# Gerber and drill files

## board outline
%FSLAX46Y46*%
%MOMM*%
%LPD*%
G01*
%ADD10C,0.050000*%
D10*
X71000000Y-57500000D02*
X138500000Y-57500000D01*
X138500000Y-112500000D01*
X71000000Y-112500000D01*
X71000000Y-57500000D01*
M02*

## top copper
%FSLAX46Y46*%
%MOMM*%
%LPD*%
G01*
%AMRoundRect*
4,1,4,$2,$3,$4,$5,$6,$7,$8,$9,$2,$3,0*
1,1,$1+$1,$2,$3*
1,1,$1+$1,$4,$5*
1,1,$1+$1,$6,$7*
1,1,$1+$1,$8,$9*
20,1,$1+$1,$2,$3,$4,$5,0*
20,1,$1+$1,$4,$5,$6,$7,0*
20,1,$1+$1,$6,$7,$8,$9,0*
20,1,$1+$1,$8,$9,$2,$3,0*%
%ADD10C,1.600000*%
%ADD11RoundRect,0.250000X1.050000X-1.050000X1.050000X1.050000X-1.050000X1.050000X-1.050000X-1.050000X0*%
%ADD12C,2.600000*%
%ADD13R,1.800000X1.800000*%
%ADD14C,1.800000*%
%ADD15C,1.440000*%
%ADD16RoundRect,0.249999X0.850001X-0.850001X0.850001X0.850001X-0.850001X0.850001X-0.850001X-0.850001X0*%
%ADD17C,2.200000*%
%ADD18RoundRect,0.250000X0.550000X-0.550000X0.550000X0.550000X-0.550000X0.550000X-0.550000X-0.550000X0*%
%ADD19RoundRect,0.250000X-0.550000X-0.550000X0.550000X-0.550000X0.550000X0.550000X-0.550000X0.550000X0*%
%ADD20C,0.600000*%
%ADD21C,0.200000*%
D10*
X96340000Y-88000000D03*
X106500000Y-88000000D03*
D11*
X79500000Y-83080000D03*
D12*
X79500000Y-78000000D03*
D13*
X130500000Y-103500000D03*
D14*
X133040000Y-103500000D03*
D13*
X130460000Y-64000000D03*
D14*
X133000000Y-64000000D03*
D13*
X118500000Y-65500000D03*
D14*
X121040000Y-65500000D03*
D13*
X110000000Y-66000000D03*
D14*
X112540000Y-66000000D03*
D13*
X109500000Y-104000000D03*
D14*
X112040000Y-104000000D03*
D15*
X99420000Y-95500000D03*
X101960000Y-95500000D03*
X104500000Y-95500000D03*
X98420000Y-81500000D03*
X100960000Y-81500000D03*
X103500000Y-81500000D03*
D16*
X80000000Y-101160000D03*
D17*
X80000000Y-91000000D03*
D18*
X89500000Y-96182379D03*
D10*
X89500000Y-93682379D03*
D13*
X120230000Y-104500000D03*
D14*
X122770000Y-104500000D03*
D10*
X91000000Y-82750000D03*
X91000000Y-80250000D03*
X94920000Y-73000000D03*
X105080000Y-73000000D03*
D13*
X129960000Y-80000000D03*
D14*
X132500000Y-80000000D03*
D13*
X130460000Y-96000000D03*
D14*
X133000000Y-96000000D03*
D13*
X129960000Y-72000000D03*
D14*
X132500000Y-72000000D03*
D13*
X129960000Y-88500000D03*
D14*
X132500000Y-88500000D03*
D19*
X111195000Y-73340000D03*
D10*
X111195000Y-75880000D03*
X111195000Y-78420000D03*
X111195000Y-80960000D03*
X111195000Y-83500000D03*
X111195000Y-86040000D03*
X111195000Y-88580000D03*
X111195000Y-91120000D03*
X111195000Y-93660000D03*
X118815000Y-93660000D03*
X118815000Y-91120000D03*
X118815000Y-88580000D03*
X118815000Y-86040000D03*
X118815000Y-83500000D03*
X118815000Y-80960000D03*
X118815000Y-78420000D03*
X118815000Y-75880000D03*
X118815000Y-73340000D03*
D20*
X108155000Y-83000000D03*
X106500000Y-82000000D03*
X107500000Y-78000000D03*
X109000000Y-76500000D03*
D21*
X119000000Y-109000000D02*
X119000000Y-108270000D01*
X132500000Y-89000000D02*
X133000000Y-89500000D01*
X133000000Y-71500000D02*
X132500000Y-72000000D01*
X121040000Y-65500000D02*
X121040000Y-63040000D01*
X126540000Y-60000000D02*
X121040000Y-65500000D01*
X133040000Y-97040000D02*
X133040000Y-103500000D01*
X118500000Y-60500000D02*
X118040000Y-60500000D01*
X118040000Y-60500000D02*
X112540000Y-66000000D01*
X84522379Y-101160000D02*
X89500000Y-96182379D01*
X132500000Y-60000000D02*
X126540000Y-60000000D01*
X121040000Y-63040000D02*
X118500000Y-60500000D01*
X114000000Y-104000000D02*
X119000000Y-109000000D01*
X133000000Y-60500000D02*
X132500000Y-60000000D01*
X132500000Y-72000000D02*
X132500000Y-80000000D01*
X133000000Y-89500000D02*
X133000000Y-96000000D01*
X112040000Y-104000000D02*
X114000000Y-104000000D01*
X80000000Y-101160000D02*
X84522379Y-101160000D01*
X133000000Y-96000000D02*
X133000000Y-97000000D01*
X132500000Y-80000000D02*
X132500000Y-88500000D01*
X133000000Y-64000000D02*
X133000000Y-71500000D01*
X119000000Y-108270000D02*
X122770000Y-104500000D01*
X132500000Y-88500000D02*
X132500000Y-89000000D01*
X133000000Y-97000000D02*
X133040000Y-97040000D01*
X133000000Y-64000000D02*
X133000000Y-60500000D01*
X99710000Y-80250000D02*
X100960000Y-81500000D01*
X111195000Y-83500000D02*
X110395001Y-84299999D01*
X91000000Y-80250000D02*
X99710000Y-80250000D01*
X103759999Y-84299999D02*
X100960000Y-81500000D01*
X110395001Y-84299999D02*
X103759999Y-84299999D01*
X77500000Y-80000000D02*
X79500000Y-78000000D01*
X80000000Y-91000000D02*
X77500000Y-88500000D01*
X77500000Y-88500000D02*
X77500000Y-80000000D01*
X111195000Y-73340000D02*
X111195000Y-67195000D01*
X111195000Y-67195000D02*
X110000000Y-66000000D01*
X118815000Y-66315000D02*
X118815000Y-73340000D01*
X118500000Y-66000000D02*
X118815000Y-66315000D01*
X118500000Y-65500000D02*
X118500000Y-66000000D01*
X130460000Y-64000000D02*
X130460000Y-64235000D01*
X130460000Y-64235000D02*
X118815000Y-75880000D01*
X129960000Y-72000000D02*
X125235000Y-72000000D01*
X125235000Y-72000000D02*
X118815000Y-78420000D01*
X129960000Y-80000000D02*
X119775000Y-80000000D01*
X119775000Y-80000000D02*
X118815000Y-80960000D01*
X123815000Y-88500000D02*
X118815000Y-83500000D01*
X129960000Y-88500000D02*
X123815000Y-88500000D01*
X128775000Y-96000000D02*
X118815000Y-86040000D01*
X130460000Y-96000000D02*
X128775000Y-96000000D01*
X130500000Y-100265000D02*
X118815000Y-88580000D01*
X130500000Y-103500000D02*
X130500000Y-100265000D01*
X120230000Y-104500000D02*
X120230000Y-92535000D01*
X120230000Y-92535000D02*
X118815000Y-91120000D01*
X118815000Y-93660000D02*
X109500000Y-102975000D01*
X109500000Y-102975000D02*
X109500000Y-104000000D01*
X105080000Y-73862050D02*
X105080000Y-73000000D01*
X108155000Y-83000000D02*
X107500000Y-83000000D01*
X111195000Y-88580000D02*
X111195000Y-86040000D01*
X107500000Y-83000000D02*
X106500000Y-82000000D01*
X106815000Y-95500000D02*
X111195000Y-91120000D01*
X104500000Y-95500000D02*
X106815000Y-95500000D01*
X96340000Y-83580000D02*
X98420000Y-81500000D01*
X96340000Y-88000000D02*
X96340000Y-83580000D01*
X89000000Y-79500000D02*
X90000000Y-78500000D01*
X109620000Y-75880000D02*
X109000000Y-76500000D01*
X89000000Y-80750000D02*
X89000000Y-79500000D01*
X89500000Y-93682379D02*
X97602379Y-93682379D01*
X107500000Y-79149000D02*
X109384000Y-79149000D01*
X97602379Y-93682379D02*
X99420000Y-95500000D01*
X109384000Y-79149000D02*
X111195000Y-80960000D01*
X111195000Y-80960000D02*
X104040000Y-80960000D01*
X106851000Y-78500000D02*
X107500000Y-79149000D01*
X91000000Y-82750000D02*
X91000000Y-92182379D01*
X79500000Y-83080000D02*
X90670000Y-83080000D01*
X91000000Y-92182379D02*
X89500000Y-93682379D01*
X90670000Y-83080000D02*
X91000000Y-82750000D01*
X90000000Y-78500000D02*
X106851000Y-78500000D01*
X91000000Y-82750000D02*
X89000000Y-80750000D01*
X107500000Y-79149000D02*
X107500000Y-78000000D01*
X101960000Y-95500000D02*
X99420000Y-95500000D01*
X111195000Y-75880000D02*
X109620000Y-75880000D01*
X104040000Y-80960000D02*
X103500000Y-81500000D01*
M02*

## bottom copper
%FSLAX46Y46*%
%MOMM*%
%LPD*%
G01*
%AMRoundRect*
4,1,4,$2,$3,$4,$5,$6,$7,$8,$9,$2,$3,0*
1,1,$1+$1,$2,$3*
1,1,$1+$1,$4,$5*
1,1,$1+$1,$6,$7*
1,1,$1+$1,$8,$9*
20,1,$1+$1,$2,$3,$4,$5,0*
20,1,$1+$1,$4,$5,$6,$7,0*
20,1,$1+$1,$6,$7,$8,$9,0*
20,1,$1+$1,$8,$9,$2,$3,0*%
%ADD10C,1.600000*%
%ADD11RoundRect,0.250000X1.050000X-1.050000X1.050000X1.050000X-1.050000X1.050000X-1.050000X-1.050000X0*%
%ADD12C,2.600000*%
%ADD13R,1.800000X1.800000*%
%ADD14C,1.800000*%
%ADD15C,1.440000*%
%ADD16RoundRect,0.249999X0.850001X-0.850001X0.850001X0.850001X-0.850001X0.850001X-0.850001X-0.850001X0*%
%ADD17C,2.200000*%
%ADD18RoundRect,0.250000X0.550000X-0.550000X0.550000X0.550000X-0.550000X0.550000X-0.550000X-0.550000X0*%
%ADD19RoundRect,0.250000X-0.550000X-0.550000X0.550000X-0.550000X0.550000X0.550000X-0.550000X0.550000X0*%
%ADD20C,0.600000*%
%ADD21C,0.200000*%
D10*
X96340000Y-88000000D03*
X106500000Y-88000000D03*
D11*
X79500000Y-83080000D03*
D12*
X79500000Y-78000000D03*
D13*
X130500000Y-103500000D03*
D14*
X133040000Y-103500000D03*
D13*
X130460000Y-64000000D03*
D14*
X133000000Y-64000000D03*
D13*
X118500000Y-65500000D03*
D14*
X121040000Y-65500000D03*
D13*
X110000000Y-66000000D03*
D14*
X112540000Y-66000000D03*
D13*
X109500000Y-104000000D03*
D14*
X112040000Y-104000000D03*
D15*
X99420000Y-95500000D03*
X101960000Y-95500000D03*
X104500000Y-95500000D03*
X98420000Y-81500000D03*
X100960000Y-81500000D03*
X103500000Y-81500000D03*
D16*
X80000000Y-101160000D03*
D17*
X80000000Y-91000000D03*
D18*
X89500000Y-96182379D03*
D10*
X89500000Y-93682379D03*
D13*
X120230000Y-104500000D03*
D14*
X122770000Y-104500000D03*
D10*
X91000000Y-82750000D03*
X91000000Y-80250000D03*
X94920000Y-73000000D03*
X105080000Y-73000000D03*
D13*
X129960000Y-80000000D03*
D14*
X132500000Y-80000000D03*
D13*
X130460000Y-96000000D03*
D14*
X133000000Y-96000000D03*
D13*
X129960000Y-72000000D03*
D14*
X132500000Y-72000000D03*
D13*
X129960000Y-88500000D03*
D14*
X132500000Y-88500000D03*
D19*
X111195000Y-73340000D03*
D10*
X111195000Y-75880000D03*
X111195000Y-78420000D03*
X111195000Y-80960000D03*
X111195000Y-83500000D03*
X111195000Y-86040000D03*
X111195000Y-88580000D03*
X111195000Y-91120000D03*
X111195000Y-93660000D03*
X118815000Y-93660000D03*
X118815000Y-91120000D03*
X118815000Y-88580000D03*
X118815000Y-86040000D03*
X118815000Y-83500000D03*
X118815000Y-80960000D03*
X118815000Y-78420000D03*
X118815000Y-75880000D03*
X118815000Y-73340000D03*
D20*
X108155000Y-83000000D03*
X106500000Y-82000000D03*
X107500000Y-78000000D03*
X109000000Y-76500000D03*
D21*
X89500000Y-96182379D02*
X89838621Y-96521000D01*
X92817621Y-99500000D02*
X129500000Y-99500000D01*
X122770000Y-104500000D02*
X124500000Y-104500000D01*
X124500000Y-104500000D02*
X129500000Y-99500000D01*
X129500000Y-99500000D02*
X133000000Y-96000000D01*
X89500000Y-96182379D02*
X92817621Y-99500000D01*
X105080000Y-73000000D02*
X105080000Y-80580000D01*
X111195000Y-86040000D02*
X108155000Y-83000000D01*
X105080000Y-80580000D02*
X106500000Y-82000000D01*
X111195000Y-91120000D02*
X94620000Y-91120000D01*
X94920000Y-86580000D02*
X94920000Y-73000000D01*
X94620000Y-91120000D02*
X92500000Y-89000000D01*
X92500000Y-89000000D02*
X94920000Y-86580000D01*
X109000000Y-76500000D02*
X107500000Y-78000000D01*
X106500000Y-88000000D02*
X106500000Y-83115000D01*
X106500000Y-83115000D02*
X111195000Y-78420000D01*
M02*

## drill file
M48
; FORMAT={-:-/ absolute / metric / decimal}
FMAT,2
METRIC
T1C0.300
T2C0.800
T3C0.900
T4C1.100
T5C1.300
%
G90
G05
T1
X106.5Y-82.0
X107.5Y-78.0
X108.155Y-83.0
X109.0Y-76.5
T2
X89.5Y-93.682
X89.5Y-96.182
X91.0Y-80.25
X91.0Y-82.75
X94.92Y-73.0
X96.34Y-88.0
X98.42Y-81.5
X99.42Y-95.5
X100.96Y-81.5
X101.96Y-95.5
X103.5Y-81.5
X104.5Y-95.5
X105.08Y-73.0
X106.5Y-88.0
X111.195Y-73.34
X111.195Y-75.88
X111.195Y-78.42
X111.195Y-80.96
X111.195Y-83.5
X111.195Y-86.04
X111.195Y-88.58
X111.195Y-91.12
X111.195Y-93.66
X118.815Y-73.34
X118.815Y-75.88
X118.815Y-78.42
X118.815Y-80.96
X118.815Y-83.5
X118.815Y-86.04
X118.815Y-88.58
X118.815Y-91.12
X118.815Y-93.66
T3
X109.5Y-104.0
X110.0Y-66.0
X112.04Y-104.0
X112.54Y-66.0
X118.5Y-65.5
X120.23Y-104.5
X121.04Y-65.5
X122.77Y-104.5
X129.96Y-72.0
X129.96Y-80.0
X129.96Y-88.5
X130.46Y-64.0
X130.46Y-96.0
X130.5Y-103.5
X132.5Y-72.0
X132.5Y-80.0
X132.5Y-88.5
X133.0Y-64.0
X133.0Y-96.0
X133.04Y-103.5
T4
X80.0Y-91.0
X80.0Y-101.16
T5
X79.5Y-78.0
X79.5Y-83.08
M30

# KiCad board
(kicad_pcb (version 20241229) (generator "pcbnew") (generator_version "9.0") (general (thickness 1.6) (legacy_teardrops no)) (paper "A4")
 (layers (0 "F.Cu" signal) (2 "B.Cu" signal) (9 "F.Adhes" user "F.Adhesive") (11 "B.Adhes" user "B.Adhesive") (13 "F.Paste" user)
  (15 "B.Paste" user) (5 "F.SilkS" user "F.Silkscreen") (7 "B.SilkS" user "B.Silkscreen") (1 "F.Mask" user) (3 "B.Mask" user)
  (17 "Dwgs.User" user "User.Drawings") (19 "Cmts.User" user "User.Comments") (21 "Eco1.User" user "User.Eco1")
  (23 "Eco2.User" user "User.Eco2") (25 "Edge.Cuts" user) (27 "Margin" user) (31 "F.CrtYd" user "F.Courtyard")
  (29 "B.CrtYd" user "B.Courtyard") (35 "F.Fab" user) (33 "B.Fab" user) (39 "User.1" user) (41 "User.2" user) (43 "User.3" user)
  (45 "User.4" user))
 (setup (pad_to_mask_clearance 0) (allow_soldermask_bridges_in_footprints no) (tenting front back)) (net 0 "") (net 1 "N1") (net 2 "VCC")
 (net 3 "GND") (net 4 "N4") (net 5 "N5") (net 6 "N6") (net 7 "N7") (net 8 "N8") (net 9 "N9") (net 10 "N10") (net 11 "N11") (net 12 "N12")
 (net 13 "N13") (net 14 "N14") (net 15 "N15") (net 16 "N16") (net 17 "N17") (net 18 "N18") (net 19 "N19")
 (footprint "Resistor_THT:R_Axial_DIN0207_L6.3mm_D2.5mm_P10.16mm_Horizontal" (layer "F.Cu") (at 96.34 88)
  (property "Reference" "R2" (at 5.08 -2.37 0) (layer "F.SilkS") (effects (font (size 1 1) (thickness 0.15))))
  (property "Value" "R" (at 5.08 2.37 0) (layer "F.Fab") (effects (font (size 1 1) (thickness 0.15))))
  (pad "1" thru_hole circle (at 0 0) (size 1.6 1.6) (drill 0.8) (layers "*.Cu" "*.Mask") (remove_unused_layers no) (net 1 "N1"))
  (pad "2" thru_hole circle (at 10.16 0) (size 1.6 1.6) (drill 0.8) (layers "*.Cu" "*.Mask") (remove_unused_layers no) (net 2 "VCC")))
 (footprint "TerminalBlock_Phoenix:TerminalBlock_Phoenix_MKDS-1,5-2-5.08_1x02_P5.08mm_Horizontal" (layer "F.Cu") (at 79.5 83.08 90)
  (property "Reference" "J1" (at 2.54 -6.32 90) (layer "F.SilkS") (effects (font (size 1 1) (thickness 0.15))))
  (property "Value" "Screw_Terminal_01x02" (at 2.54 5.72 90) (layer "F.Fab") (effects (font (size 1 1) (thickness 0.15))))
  (pad "1" thru_hole roundrect (at 0 0 90) (size 2.6 2.6) (drill 1.3) (layers "*.Cu" "*.Mask") (remove_unused_layers no)
   (roundrect_rratio 0.096154) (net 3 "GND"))
  (pad "2" thru_hole circle (at 5.08 0 90) (size 2.6 2.6) (drill 1.3) (layers "*.Cu" "*.Mask") (remove_unused_layers no) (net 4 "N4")))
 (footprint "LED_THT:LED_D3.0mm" (layer "F.Cu") (at 130.5 103.5)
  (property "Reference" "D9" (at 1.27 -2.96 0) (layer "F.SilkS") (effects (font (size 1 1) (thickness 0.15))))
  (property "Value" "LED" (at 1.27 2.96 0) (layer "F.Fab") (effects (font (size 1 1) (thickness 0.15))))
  (pad "1" thru_hole rect (at 0 0) (size 1.8 1.8) (drill 0.9) (layers "*.Cu" "*.Mask") (remove_unused_layers no) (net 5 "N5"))
  (pad "2" thru_hole circle (at 2.54 0) (size 1.8 1.8) (drill 0.9) (layers "*.Cu" "*.Mask") (remove_unused_layers no) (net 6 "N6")))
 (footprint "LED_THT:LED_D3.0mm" (layer "F.Cu") (at 130.46 64)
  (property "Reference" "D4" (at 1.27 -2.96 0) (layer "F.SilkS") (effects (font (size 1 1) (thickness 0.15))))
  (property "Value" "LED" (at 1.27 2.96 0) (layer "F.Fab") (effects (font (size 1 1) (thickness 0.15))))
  (pad "1" thru_hole rect (at 0 0) (size 1.8 1.8) (drill 0.9) (layers "*.Cu" "*.Mask") (remove_unused_layers no) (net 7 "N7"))
  (pad "2" thru_hole circle (at 2.54 0) (size 1.8 1.8) (drill 0.9) (layers "*.Cu" "*.Mask") (remove_unused_layers no) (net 6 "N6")))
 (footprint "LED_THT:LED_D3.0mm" (layer "F.Cu") (at 118.5 65.5)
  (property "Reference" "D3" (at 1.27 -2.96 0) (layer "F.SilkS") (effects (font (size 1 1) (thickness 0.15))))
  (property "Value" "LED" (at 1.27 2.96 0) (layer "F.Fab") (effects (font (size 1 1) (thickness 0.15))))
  (pad "1" thru_hole rect (at 0 0) (size 1.8 1.8) (drill 0.9) (layers "*.Cu" "*.Mask") (remove_unused_layers no) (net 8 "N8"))
  (pad "2" thru_hole circle (at 2.54 0) (size 1.8 1.8) (drill 0.9) (layers "*.Cu" "*.Mask") (remove_unused_layers no) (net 6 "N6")))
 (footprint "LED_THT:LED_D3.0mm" (layer "F.Cu") (at 110 66)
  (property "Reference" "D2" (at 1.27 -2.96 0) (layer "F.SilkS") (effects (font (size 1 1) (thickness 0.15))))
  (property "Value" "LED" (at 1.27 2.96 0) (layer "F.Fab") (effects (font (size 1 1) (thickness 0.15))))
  (pad "1" thru_hole rect (at 0 0) (size 1.8 1.8) (drill 0.9) (layers "*.Cu" "*.Mask") (remove_unused_layers no) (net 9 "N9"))
  (pad "2" thru_hole circle (at 2.54 0) (size 1.8 1.8) (drill 0.9) (layers "*.Cu" "*.Mask") (remove_unused_layers no) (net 6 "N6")))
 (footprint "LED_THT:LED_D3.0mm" (layer "F.Cu") (at 109.5 104)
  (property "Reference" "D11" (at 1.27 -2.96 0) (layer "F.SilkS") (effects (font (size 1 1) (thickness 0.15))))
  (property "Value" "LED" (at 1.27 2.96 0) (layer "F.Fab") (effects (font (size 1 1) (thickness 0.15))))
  (pad "1" thru_hole rect (at 0 0) (size 1.8 1.8) (drill 0.9) (layers "*.Cu" "*.Mask") (remove_unused_layers no) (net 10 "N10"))
  (pad "2" thru_hole circle (at 2.54 0) (size 1.8 1.8) (drill 0.9) (layers "*.Cu" "*.Mask") (remove_unused_layers no) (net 6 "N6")))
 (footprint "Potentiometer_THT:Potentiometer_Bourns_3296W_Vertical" (layer "F.Cu") (at 99.42 95.5 180)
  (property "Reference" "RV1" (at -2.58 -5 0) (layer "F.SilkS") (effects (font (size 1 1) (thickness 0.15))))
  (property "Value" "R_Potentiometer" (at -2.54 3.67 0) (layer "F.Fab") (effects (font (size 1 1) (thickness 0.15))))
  (pad "1" thru_hole circle (at 0 0 180) (size 1.44 1.44) (drill 0.8) (layers "*.Cu" "*.Mask") (remove_unused_layers no) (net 3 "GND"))
  (pad "2" thru_hole circle (at -2.54 0 180) (size 1.44 1.44) (drill 0.8) (layers "*.Cu" "*.Mask") (remove_unused_layers no) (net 3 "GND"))
  (pad "3" thru_hole circle (at -5.08 0 180) (size 1.44 1.44) (drill 0.8) (layers "*.Cu" "*.Mask") (remove_unused_layers no) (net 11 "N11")))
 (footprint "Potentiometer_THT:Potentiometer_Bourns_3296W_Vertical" (layer "F.Cu") (at 98.42 81.5 180)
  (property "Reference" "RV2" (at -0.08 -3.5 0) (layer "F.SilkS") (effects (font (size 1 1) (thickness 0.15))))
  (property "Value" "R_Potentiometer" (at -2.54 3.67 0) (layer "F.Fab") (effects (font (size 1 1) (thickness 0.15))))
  (pad "1" thru_hole circle (at 0 0 180) (size 1.44 1.44) (drill 0.8) (layers "*.Cu" "*.Mask") (remove_unused_layers no) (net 1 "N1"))
  (pad "2" thru_hole circle (at -2.54 0 180) (size 1.44 1.44) (drill 0.8) (layers "*.Cu" "*.Mask") (remove_unused_layers no) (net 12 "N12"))
  (pad "3" thru_hole circle (at -5.08 0 180) (size 1.44 1.44) (drill 0.8) (layers "*.Cu" "*.Mask") (remove_unused_layers no) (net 3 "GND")))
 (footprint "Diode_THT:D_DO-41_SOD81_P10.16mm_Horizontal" (layer "F.Cu") (at 80 101.16 90)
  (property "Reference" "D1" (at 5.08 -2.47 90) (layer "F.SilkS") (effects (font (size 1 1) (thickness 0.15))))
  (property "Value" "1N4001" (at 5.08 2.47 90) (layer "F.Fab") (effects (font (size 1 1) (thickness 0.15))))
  (pad "1" thru_hole roundrect (at 0 0 90) (size 2.2 2.2) (drill 1.1) (layers "*.Cu" "*.Mask") (remove_unused_layers no)
   (roundrect_rratio 0.113636) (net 6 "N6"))
  (pad "2" thru_hole circle (at 10.16 0 90) (size 2.2 2.2) (drill 1.1) (layers "*.Cu" "*.Mask") (remove_unused_layers no) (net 4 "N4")))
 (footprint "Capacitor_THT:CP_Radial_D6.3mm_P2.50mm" (layer "F.Cu") (at 89.5 96.182379 90)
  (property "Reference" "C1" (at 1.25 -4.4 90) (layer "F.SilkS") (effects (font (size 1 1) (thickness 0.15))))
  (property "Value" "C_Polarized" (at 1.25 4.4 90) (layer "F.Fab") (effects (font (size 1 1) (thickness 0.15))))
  (pad "1" thru_hole roundrect (at 0 0 90) (size 1.6 1.6) (drill 0.8) (layers "*.Cu" "*.Mask") (remove_unused_layers no)
   (roundrect_rratio 0.15625) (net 6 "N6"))
  (pad "2" thru_hole circle (at 2.5 0 90) (size 1.6 1.6) (drill 0.8) (layers "*.Cu" "*.Mask") (remove_unused_layers no) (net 3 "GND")))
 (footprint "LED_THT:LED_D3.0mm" (layer "F.Cu") (at 120.23 104.5)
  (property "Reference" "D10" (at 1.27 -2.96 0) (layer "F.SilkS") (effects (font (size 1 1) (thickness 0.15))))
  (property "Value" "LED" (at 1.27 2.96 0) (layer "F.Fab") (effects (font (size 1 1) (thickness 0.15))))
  (pad "1" thru_hole rect (at 0 0) (size 1.8 1.8) (drill 0.9) (layers "*.Cu" "*.Mask") (remove_unused_layers no) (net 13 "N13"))
  (pad "2" thru_hole circle (at 2.54 0) (size 1.8 1.8) (drill 0.9) (layers "*.Cu" "*.Mask") (remove_unused_layers no) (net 6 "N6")))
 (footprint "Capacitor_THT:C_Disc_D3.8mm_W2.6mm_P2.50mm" (layer "F.Cu") (at 91 82.75 90)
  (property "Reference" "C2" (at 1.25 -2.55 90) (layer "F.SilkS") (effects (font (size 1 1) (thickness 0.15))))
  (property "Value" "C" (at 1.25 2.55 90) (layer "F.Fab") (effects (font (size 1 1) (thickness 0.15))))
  (pad "1" thru_hole circle (at 0 0 90) (size 1.6 1.6) (drill 0.8) (layers "*.Cu" "*.Mask") (remove_unused_layers no) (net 3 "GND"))
  (pad "2" thru_hole circle (at 2.5 0 90) (size 1.6 1.6) (drill 0.8) (layers "*.Cu" "*.Mask") (remove_unused_layers no) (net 12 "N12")))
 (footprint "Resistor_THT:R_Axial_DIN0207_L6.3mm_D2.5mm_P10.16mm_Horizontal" (layer "F.Cu") (at 94.92 73)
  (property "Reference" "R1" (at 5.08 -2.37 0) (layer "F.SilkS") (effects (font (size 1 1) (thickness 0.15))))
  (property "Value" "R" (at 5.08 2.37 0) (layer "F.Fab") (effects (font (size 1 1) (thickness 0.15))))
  (pad "1" thru_hole circle (at 0 0) (size 1.6 1.6) (drill 0.8) (layers "*.Cu" "*.Mask") (remove_unused_layers no) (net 11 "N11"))
  (pad "2" thru_hole circle (at 10.16 0) (size 1.6 1.6) (drill 0.8) (layers "*.Cu" "*.Mask") (remove_unused_layers no) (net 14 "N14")))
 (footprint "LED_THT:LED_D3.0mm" (layer "F.Cu") (at 129.96 80)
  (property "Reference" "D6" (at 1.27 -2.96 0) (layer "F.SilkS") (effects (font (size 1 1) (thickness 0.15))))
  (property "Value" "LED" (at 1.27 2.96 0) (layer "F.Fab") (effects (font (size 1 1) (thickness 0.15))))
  (pad "1" thru_hole rect (at 0 0) (size 1.8 1.8) (drill 0.9) (layers "*.Cu" "*.Mask") (remove_unused_layers no) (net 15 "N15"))
  (pad "2" thru_hole circle (at 2.54 0) (size 1.8 1.8) (drill 0.9) (layers "*.Cu" "*.Mask") (remove_unused_layers no) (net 6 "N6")))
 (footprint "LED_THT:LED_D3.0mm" (layer "F.Cu") (at 130.46 96)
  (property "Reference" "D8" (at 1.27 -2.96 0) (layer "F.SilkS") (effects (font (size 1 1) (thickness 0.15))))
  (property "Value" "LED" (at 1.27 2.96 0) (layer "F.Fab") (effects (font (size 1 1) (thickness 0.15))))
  (pad "1" thru_hole rect (at 0 0) (size 1.8 1.8) (drill 0.9) (layers "*.Cu" "*.Mask") (remove_unused_layers no) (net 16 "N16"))
  (pad "2" thru_hole circle (at 2.54 0) (size 1.8 1.8) (drill 0.9) (layers "*.Cu" "*.Mask") (remove_unused_layers no) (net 6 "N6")))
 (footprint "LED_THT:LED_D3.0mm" (layer "F.Cu") (at 129.96 72)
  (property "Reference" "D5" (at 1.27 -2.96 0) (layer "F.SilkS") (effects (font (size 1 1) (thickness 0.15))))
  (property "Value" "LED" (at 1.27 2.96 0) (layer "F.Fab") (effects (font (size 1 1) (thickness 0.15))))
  (pad "1" thru_hole rect (at 0 0) (size 1.8 1.8) (drill 0.9) (layers "*.Cu" "*.Mask") (remove_unused_layers no) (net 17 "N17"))
  (pad "2" thru_hole circle (at 2.54 0) (size 1.8 1.8) (drill 0.9) (layers "*.Cu" "*.Mask") (remove_unused_layers no) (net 6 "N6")))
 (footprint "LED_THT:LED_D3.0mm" (layer "F.Cu") (at 129.96 88.5)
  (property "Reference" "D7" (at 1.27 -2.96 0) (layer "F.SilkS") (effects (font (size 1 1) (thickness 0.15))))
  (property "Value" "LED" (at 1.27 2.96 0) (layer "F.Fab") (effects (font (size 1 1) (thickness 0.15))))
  (pad "1" thru_hole rect (at 0 0) (size 1.8 1.8) (drill 0.9) (layers "*.Cu" "*.Mask") (remove_unused_layers no) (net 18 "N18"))
  (pad "2" thru_hole circle (at 2.54 0) (size 1.8 1.8) (drill 0.9) (layers "*.Cu" "*.Mask") (remove_unused_layers no) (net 6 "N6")))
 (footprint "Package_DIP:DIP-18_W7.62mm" (layer "F.Cu") (at 111.195 73.34)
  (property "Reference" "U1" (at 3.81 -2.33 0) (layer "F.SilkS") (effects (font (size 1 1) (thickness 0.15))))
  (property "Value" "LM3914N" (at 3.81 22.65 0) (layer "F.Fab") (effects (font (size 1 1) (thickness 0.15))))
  (pad "1" thru_hole roundrect (at 0 0) (size 1.6 1.6) (drill 0.8) (layers "*.Cu" "*.Mask") (remove_unused_layers no)
   (roundrect_rratio 0.15625) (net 9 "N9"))
  (pad "2" thru_hole circle (at 0 2.54) (size 1.6 1.6) (drill 0.8) (layers "*.Cu" "*.Mask") (remove_unused_layers no) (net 3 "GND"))
  (pad "3" thru_hole circle (at 0 5.08) (size 1.6 1.6) (drill 0.8) (layers "*.Cu" "*.Mask") (remove_unused_layers no) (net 2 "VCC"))
  (pad "4" thru_hole circle (at 0 7.62) (size 1.6 1.6) (drill 0.8) (layers "*.Cu" "*.Mask") (remove_unused_layers no) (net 3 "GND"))
  (pad "5" thru_hole circle (at 0 10.16) (size 1.6 1.6) (drill 0.8) (layers "*.Cu" "*.Mask") (remove_unused_layers no) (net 12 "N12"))
  (pad "6" thru_hole circle (at 0 12.7) (size 1.6 1.6) (drill 0.8) (layers "*.Cu" "*.Mask") (remove_unused_layers no) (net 14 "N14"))
  (pad "7" thru_hole circle (at 0 15.24) (size 1.6 1.6) (drill 0.8) (layers "*.Cu" "*.Mask") (remove_unused_layers no) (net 14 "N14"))
  (pad "8" thru_hole circle (at 0 17.78) (size 1.6 1.6) (drill 0.8) (layers "*.Cu" "*.Mask") (remove_unused_layers no) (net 11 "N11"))
  (pad "9" thru_hole circle (at 0 20.32) (size 1.6 1.6) (drill 0.8) (layers "*.Cu" "*.Mask") (remove_unused_layers no) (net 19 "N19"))
  (pad "10" thru_hole circle (at 7.62 20.32) (size 1.6 1.6) (drill 0.8) (layers "*.Cu" "*.Mask") (remove_unused_layers no) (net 10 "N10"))
  (pad "11" thru_hole circle (at 7.62 17.78) (size 1.6 1.6) (drill 0.8) (layers "*.Cu" "*.Mask") (remove_unused_layers no) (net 13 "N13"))
  (pad "12" thru_hole circle (at 7.62 15.24) (size 1.6 1.6) (drill 0.8) (layers "*.Cu" "*.Mask") (remove_unused_layers no) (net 5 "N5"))
  (pad "13" thru_hole circle (at 7.62 12.7) (size 1.6 1.6) (drill 0.8) (layers "*.Cu" "*.Mask") (remove_unused_layers no) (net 16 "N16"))
  (pad "14" thru_hole circle (at 7.62 10.16) (size 1.6 1.6) (drill 0.8) (layers "*.Cu" "*.Mask") (remove_unused_layers no) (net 18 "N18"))
  (pad "15" thru_hole circle (at 7.62 7.62) (size 1.6 1.6) (drill 0.8) (layers "*.Cu" "*.Mask") (remove_unused_layers no) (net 15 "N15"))
  (pad "16" thru_hole circle (at 7.62 5.08) (size 1.6 1.6) (drill 0.8) (layers "*.Cu" "*.Mask") (remove_unused_layers no) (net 17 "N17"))
  (pad "17" thru_hole circle (at 7.62 2.54) (size 1.6 1.6) (drill 0.8) (layers "*.Cu" "*.Mask") (remove_unused_layers no) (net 7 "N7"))
  (pad "18" thru_hole circle (at 7.62 0) (size 1.6 1.6) (drill 0.8) (layers "*.Cu" "*.Mask") (remove_unused_layers no) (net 8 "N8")))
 (gr_rect (start 71 57.5) (end 138.5 112.5) (stroke (width 0.05) (type default)) (fill no) (layer "Edge.Cuts"))
 (segment (start 119 109) (end 119 108.27) (width 0.2) (layer "F.Cu") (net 6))
 (segment (start 132.5 89) (end 133 89.5) (width 0.2) (layer "F.Cu") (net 6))
 (segment (start 133 71.5) (end 132.5 72) (width 0.2) (layer "F.Cu") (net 6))
 (segment (start 121.04 65.5) (end 121.04 63.04) (width 0.2) (layer "F.Cu") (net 6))
 (segment (start 126.54 60) (end 121.04 65.5) (width 0.2) (layer "F.Cu") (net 6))
 (segment (start 133.04 97.04) (end 133.04 103.5) (width 0.2) (layer "F.Cu") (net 6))
 (segment (start 118.5 60.5) (end 118.04 60.5) (width 0.2) (layer "F.Cu") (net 6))
 (segment (start 118.04 60.5) (end 112.54 66) (width 0.2) (layer "F.Cu") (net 6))
 (segment (start 84.522379 101.16) (end 89.5 96.182379) (width 0.2) (layer "F.Cu") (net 6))
 (segment (start 132.5 60) (end 126.54 60) (width 0.2) (layer "F.Cu") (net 6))
 (segment (start 121.04 63.04) (end 118.5 60.5) (width 0.2) (layer "F.Cu") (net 6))
 (segment (start 114 104) (end 119 109) (width 0.2) (layer "F.Cu") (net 6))
 (segment (start 133 60.5) (end 132.5 60) (width 0.2) (layer "F.Cu") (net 6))
 (segment (start 132.5 72) (end 132.5 80) (width 0.2) (layer "F.Cu") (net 6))
 (segment (start 133 89.5) (end 133 96) (width 0.2) (layer "F.Cu") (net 6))
 (segment (start 112.04 104) (end 114 104) (width 0.2) (layer "F.Cu") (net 6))
 (segment (start 80 101.16) (end 84.522379 101.16) (width 0.2) (layer "F.Cu") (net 6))
 (segment (start 133 96) (end 133 97) (width 0.2) (layer "F.Cu") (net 6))
 (segment (start 132.5 80) (end 132.5 88.5) (width 0.2) (layer "F.Cu") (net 6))
 (segment (start 133 64) (end 133 71.5) (width 0.2) (layer "F.Cu") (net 6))
 (segment (start 119 108.27) (end 122.77 104.5) (width 0.2) (layer "F.Cu") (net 6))
 (segment (start 132.5 88.5) (end 132.5 89) (width 0.2) (layer "F.Cu") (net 6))
 (segment (start 133 97) (end 133.04 97.04) (width 0.2) (layer "F.Cu") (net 6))
 (segment (start 133 64) (end 133 60.5) (width 0.2) (layer "F.Cu") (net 6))
 (segment (start 89.5 96.182379) (end 89.838621 96.521) (width 0.2) (layer "B.Cu") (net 6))
 (segment (start 92.817621 99.5) (end 129.5 99.5) (width 0.2) (layer "B.Cu") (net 6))
 (segment (start 122.77 104.5) (end 124.5 104.5) (width 0.2) (layer "B.Cu") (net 6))
 (segment (start 124.5 104.5) (end 129.5 99.5) (width 0.2) (layer "B.Cu") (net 6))
 (segment (start 129.5 99.5) (end 133 96) (width 0.2) (layer "B.Cu") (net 6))
 (segment (start 89.5 96.182379) (end 92.817621 99.5) (width 0.2) (layer "B.Cu") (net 6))
 (segment (start 99.71 80.25) (end 100.96 81.5) (width 0.2) (layer "F.Cu") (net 12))
 (segment (start 111.195 83.5) (end 110.395001 84.299999) (width 0.2) (layer "F.Cu") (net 12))
 (segment (start 91 80.25) (end 99.71 80.25) (width 0.2) (layer "F.Cu") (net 12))
 (segment (start 103.759999 84.299999) (end 100.96 81.5) (width 0.2) (layer "F.Cu") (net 12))
 (segment (start 110.395001 84.299999) (end 103.759999 84.299999) (width 0.2) (layer "F.Cu") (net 12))
 (segment (start 77.5 80) (end 79.5 78) (width 0.2) (layer "F.Cu") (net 4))
 (segment (start 80 91) (end 77.5 88.5) (width 0.2) (layer "F.Cu") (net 4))
 (segment (start 77.5 88.5) (end 77.5 80) (width 0.2) (layer "F.Cu") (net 4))
 (segment (start 111.195 73.34) (end 111.195 67.195) (width 0.2) (layer "F.Cu") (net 9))
 (segment (start 111.195 67.195) (end 110 66) (width 0.2) (layer "F.Cu") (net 9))
 (segment (start 118.815 66.315) (end 118.815 73.34) (width 0.2) (layer "F.Cu") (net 8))
 (segment (start 118.5 66) (end 118.815 66.315) (width 0.2) (layer "F.Cu") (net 8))
 (segment (start 118.5 65.5) (end 118.5 66) (width 0.2) (layer "F.Cu") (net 8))
 (segment (start 130.46 64) (end 130.46 64.235) (width 0.2) (layer "F.Cu") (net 7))
 (segment (start 130.46 64.235) (end 118.815 75.88) (width 0.2) (layer "F.Cu") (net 7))
 (segment (start 129.96 72) (end 125.235 72) (width 0.2) (layer "F.Cu") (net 17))
 (segment (start 125.235 72) (end 118.815 78.42) (width 0.2) (layer "F.Cu") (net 17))
 (segment (start 129.96 80) (end 119.775 80) (width 0.2) (layer "F.Cu") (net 15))
 (segment (start 119.775 80) (end 118.815 80.96) (width 0.2) (layer "F.Cu") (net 15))
 (segment (start 123.815 88.5) (end 118.815 83.5) (width 0.2) (layer "F.Cu") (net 18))
 (segment (start 129.96 88.5) (end 123.815 88.5) (width 0.2) (layer "F.Cu") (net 18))
 (segment (start 128.775 96) (end 118.815 86.04) (width 0.2) (layer "F.Cu") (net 16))
 (segment (start 130.46 96) (end 128.775 96) (width 0.2) (layer "F.Cu") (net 16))
 (segment (start 130.5 100.265) (end 118.815 88.58) (width 0.2) (layer "F.Cu") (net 5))
 (segment (start 130.5 103.5) (end 130.5 100.265) (width 0.2) (layer "F.Cu") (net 5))
 (segment (start 120.23 104.5) (end 120.23 92.535) (width 0.2) (layer "F.Cu") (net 13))
 (segment (start 120.23 92.535) (end 118.815 91.12) (width 0.2) (layer "F.Cu") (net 13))
 (segment (start 118.815 93.66) (end 109.5 102.975) (width 0.2) (layer "F.Cu") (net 10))
 (segment (start 109.5 102.975) (end 109.5 104) (width 0.2) (layer "F.Cu") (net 10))
 (segment (start 105.08 73.86205) (end 105.08 73) (width 0.2) (layer "F.Cu") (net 14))
 (segment (start 108.155 83) (end 107.5 83) (width 0.2) (layer "F.Cu") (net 14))
 (segment (start 111.195 88.58) (end 111.195 86.04) (width 0.2) (layer "F.Cu") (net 14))
 (segment (start 107.5 83) (end 106.5 82) (width 0.2) (layer "F.Cu") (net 14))
 (via (at 108.155 83) (size 0.6) (drill 0.3) (layers "F.Cu" "B.Cu") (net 14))
 (via (at 106.5 82) (size 0.6) (drill 0.3) (layers "F.Cu" "B.Cu") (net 14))
 (segment (start 105.08 73) (end 105.08 80.58) (width 0.2) (layer "B.Cu") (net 14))
 (segment (start 111.195 86.04) (end 108.155 83) (width 0.2) (layer "B.Cu") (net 14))
 (segment (start 105.08 80.58) (end 106.5 82) (width 0.2) (layer "B.Cu") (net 14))
 (segment (start 106.815 95.5) (end 111.195 91.12) (width 0.2) (layer "F.Cu") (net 11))
 (segment (start 104.5 95.5) (end 106.815 95.5) (width 0.2) (layer "F.Cu") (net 11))
 (segment (start 111.195 91.12) (end 94.62 91.12) (width 0.2) (layer "B.Cu") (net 11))
 (segment (start 94.92 86.58) (end 94.92 73) (width 0.2) (layer "B.Cu") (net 11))
 (segment (start 94.62 91.12) (end 92.5 89) (width 0.2) (layer "B.Cu") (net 11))
 (segment (start 92.5 89) (end 94.92 86.58) (width 0.2) (layer "B.Cu") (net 11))
 (segment (start 96.34 83.58) (end 98.42 81.5) (width 0.2) (layer "F.Cu") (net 1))
 (segment (start 96.34 88) (end 96.34 83.58) (width 0.2) (layer "F.Cu") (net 1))
 (segment (start 89 79.5) (end 90 78.5) (width 0.2) (layer "F.Cu") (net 3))
 (segment (start 109.62 75.88) (end 109 76.5) (width 0.2) (layer "F.Cu") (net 3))
 (segment (start 89 80.75) (end 89 79.5) (width 0.2) (layer "F.Cu") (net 3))
 (segment (start 89.5 93.682379) (end 97.602379 93.682379) (width 0.2) (layer "F.Cu") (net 3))
 (segment (start 107.5 79.149) (end 109.384 79.149) (width 0.2) (layer "F.Cu") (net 3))
 (segment (start 97.602379 93.682379) (end 99.42 95.5) (width 0.2) (layer "F.Cu") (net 3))
 (segment (start 109.384 79.149) (end 111.195 80.96) (width 0.2) (layer "F.Cu") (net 3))
 (segment (start 111.195 80.96) (end 104.04 80.96) (width 0.2) (layer "F.Cu") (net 3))
 (segment (start 106.851 78.5) (end 107.5 79.149) (width 0.2) (layer "F.Cu") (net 3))
 (segment (start 91 82.75) (end 91 92.182379) (width 0.2) (layer "F.Cu") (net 3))
 (segment (start 79.5 83.08) (end 90.67 83.08) (width 0.2) (layer "F.Cu") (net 3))
 (segment (start 91 92.182379) (end 89.5 93.682379) (width 0.2) (layer "F.Cu") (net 3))
 (segment (start 90.67 83.08) (end 91 82.75) (width 0.2) (layer "F.Cu") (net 3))
 (segment (start 90 78.5) (end 106.851 78.5) (width 0.2) (layer "F.Cu") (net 3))
 (segment (start 91 82.75) (end 89 80.75) (width 0.2) (layer "F.Cu") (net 3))
 (segment (start 107.5 79.149) (end 107.5 78) (width 0.2) (layer "F.Cu") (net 3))
 (segment (start 101.96 95.5) (end 99.42 95.5) (width 0.2) (layer "F.Cu") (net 3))
 (segment (start 111.195 75.88) (end 109.62 75.88) (width 0.2) (layer "F.Cu") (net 3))
 (segment (start 104.04 80.96) (end 103.5 81.5) (width 0.2) (layer "F.Cu") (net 3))
 (via (at 107.5 78) (size 0.6) (drill 0.3) (layers "F.Cu" "B.Cu") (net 3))
 (via (at 109 76.5) (size 0.6) (drill 0.3) (layers "F.Cu" "B.Cu") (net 3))
 (segment (start 109 76.5) (end 107.5 78) (width 0.2) (layer "B.Cu") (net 3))
 (segment (start 106.5 88) (end 106.5 83.115) (width 0.2) (layer "B.Cu") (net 2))
 (segment (start 106.5 83.115) (end 111.195 78.42) (width 0.2) (layer "B.Cu") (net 2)))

